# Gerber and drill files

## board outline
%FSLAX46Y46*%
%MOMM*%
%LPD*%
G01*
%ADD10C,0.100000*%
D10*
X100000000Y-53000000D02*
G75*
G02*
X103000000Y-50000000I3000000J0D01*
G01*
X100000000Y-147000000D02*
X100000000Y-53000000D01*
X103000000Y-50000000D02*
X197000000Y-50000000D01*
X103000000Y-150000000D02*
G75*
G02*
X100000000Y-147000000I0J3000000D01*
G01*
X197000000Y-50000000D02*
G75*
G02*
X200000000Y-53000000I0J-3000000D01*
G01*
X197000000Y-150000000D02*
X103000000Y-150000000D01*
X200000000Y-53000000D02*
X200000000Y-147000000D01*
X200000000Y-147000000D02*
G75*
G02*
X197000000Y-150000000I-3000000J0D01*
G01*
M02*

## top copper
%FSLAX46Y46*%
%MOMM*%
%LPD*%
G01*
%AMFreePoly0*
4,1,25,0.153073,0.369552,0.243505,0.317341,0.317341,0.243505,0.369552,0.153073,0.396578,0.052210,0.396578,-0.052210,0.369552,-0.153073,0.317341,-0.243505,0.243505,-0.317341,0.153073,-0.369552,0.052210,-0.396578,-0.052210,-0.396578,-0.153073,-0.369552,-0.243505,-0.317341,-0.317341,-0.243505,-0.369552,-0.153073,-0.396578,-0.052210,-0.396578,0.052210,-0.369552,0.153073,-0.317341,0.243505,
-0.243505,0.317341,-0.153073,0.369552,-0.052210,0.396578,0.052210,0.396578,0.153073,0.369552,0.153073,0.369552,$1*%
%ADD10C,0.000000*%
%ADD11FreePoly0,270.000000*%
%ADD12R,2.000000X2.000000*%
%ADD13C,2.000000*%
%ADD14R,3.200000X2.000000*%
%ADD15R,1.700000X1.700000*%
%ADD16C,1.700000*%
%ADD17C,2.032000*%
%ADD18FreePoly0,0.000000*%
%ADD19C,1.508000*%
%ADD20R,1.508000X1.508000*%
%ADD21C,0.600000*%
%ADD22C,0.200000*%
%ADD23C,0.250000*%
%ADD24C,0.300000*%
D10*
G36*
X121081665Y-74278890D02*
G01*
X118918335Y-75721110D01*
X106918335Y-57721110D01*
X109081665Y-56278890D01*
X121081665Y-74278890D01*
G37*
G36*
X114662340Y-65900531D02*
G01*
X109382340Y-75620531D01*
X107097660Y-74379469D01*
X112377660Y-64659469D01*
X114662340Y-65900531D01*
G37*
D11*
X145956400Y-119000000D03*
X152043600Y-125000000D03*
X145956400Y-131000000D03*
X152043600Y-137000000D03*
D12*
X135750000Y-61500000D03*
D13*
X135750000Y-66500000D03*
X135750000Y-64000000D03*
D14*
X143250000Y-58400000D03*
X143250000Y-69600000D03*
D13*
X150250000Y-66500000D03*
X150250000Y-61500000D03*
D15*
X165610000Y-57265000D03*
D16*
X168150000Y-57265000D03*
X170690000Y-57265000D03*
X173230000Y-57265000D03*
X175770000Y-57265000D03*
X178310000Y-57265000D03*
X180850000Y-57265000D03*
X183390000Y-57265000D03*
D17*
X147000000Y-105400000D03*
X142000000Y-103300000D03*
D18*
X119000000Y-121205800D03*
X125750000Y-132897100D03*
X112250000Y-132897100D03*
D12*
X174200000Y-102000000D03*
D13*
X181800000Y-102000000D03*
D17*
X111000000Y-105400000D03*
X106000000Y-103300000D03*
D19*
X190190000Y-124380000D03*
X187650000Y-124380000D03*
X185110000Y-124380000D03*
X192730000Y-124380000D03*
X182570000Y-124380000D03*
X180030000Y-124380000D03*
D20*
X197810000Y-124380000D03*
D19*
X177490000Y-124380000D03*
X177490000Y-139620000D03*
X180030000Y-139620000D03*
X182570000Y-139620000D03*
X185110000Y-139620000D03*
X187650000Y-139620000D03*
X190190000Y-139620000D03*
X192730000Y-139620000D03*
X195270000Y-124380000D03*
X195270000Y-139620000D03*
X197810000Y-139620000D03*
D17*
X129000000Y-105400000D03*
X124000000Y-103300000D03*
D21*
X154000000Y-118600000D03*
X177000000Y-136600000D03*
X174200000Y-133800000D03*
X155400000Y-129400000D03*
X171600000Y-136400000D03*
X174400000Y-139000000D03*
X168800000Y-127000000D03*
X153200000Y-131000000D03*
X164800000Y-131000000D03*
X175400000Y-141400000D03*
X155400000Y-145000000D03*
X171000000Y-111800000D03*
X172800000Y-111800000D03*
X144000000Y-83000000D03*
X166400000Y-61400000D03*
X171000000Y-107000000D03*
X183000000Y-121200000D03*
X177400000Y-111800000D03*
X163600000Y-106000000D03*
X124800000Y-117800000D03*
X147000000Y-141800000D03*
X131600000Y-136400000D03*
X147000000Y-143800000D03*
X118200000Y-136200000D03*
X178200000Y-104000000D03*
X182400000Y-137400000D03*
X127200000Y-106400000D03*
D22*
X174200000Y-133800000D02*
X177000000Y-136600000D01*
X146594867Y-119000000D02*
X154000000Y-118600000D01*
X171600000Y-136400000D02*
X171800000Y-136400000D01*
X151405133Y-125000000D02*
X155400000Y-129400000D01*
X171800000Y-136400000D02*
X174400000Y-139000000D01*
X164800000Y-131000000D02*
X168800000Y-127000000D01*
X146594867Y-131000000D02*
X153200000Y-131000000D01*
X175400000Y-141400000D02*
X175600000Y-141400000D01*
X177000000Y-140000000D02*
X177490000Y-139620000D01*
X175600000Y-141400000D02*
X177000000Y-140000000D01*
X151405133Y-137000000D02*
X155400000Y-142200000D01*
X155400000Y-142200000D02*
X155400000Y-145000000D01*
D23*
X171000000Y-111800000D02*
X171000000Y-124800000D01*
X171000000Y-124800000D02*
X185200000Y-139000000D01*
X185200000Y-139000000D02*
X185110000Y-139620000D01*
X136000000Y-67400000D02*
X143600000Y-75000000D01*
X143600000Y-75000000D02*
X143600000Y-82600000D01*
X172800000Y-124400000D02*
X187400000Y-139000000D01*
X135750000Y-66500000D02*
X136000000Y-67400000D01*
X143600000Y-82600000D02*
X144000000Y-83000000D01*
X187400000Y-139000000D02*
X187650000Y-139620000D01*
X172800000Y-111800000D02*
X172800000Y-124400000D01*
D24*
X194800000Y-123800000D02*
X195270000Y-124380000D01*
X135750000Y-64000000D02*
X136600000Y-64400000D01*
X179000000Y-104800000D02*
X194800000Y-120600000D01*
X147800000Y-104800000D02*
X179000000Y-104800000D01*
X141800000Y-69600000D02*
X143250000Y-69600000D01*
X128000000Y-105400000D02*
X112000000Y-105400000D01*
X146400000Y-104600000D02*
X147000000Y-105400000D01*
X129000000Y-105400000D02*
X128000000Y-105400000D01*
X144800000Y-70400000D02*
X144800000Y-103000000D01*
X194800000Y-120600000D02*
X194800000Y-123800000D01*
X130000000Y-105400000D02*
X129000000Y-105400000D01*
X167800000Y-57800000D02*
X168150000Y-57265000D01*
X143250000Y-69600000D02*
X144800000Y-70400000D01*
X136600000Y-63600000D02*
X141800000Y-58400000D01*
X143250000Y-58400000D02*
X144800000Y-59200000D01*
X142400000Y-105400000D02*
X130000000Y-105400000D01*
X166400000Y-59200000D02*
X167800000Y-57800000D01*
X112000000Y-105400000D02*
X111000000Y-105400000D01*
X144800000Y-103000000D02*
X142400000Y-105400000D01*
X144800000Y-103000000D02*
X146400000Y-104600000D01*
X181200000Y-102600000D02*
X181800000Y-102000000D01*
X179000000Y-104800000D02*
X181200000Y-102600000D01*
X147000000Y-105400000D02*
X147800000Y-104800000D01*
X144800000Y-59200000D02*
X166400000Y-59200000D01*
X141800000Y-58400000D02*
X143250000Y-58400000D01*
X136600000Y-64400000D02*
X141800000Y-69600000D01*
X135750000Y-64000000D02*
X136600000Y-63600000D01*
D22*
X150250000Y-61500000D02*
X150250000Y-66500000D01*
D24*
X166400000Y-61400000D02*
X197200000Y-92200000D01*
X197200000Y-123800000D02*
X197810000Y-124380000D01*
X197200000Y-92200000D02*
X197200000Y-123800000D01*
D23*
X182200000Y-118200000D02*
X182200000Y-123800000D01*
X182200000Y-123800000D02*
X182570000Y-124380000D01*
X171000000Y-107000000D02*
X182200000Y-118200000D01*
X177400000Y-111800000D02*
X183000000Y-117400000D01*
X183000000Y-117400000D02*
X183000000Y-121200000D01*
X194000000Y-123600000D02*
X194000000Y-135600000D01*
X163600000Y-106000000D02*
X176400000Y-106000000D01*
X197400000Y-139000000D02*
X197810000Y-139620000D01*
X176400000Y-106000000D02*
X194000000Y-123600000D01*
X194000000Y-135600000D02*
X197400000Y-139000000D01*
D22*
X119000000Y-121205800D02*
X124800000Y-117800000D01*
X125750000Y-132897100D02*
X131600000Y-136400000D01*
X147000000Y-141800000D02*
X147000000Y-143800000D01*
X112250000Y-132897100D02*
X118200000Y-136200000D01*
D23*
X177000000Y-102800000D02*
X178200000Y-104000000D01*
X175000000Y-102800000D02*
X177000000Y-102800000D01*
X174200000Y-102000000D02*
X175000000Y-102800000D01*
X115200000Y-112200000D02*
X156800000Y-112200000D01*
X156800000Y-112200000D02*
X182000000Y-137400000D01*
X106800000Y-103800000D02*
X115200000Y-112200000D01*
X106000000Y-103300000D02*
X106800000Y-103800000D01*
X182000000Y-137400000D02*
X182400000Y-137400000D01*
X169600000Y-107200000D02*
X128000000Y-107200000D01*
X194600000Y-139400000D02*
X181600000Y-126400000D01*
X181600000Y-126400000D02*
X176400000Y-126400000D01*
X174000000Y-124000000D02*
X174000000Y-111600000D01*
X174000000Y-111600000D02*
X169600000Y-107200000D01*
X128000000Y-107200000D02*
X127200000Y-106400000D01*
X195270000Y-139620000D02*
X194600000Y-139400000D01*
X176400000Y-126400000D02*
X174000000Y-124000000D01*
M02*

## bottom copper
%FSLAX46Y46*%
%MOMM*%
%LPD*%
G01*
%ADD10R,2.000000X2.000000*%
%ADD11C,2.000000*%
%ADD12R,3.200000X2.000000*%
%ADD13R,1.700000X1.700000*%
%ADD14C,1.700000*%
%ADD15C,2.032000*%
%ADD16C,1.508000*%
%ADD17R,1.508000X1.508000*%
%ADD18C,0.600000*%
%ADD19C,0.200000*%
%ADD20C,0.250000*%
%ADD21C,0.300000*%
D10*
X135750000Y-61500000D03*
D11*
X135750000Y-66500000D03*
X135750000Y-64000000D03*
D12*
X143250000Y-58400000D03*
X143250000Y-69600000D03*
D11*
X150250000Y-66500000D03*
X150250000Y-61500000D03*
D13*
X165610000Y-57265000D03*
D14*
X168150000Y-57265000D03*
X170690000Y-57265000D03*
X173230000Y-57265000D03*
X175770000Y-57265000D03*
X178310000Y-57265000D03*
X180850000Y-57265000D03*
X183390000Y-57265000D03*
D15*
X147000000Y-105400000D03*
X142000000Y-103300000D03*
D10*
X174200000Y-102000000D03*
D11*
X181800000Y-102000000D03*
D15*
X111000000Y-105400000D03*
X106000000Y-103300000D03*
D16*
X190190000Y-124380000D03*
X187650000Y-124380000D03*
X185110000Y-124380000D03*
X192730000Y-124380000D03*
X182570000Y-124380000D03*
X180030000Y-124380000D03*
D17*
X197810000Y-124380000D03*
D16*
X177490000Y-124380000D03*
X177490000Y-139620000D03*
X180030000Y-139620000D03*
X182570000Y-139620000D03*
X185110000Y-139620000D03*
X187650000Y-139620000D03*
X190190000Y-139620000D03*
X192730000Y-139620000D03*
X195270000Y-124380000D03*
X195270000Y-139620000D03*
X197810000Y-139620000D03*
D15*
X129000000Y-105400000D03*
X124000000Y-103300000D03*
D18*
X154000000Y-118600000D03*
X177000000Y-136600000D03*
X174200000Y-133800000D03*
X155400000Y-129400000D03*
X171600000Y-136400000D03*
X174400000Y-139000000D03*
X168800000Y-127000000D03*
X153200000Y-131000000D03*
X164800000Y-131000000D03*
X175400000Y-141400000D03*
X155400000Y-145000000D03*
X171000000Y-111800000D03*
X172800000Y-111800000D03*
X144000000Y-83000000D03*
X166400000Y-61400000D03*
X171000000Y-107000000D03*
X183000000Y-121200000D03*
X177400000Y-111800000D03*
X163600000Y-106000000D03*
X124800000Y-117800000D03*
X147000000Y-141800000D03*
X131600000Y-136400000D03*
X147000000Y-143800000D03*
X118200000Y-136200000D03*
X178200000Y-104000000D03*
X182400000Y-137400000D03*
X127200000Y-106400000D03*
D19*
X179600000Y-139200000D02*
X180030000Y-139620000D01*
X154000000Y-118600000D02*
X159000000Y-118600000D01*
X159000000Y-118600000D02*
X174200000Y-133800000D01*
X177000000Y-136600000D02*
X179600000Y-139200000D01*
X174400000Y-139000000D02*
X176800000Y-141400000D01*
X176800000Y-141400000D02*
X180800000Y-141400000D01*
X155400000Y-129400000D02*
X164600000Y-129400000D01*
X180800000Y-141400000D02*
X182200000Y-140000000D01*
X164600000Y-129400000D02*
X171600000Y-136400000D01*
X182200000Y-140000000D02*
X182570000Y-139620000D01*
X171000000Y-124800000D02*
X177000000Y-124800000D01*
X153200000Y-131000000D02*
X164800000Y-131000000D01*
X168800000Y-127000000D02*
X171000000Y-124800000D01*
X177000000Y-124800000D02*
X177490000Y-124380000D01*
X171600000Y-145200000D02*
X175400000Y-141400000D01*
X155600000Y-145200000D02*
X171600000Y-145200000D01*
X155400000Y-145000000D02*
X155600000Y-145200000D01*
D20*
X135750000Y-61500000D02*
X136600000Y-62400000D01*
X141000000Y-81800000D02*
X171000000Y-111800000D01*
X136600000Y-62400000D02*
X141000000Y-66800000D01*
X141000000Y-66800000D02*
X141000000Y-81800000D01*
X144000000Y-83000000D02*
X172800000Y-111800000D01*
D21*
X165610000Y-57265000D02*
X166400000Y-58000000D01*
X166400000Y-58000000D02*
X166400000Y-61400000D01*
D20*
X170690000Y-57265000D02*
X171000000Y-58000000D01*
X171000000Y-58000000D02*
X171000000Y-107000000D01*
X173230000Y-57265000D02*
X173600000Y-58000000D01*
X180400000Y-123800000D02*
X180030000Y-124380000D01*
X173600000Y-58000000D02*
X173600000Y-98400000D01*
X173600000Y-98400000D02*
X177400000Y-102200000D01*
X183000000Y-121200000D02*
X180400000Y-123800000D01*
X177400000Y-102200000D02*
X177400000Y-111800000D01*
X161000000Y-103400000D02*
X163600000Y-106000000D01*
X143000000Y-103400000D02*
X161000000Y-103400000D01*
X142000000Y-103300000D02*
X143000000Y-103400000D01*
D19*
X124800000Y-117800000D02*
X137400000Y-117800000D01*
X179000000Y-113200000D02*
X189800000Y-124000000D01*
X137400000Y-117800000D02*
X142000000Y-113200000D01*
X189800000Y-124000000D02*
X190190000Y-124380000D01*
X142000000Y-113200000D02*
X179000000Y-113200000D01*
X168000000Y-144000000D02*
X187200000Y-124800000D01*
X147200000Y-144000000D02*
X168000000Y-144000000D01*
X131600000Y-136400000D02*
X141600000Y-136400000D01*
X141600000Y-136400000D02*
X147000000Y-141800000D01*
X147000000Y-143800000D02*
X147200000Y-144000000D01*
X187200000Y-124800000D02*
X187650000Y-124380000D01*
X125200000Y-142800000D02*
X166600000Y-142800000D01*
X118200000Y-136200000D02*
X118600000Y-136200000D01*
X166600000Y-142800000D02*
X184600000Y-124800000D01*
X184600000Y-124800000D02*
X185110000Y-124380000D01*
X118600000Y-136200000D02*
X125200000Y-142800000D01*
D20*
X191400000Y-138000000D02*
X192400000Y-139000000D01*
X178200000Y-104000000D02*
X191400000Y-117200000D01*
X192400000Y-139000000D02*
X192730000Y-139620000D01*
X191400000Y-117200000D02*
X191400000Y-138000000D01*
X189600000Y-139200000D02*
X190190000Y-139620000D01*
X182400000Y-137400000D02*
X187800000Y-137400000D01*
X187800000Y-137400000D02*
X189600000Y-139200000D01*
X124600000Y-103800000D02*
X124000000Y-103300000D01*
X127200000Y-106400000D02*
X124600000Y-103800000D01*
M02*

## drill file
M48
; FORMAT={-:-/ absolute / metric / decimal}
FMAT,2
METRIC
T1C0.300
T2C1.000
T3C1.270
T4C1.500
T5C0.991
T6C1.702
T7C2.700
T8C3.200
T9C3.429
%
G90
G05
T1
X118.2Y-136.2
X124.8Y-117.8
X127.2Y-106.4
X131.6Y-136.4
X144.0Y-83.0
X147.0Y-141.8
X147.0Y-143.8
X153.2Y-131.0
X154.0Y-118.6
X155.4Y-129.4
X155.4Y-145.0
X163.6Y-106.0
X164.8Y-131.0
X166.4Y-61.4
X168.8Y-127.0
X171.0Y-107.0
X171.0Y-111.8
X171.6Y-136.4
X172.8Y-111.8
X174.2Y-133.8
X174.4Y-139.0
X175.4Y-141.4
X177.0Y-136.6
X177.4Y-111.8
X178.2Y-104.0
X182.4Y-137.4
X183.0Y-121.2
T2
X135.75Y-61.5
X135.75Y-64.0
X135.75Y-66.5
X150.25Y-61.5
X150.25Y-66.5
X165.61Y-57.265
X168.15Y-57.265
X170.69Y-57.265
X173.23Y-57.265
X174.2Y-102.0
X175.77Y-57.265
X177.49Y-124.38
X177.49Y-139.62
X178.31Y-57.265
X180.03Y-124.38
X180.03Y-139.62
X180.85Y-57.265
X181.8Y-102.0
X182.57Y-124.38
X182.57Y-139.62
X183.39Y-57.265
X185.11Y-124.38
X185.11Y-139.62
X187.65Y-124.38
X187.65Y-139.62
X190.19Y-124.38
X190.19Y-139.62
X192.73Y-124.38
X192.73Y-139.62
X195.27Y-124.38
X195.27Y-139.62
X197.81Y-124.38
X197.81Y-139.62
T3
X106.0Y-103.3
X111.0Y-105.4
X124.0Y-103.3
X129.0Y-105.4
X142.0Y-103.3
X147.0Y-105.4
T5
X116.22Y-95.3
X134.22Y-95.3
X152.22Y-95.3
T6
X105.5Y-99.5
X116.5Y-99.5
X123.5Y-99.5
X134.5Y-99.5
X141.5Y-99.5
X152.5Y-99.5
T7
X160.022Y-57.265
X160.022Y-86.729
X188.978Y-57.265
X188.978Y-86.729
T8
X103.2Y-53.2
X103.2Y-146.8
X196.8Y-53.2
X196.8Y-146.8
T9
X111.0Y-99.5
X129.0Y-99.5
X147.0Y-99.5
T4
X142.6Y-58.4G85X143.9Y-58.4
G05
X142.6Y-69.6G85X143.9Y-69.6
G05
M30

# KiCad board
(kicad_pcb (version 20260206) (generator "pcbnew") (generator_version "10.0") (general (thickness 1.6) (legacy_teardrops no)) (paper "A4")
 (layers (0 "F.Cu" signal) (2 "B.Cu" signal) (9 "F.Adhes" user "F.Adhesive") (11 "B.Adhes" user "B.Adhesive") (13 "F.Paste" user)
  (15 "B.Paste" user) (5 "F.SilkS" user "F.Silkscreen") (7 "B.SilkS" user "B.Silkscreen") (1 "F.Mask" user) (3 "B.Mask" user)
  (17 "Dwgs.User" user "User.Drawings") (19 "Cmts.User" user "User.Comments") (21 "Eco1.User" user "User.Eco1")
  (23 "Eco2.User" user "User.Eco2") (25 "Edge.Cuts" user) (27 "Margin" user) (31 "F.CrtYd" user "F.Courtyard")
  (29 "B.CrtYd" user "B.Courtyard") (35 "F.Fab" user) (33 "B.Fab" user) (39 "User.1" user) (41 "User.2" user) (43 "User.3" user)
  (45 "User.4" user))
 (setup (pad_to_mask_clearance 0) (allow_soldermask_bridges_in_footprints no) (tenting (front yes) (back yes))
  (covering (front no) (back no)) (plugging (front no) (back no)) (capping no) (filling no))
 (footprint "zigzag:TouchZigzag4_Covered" (layer "F.Cu") (at 149 128 -90)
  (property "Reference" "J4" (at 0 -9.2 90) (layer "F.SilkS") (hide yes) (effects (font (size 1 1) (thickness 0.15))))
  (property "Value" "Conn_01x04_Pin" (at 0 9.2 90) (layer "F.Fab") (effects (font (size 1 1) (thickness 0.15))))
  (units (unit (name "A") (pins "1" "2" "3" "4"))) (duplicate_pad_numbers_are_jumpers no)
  (pad "1" smd custom (at -9 3.0436 270) (size 0.8 0.8) (layers "F.Cu") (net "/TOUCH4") (options (clearance outline) (anchor circle))
   (primitives))
  (pad "2" smd custom (at -3 -3.0436 270) (size 0.8 0.8) (layers "F.Cu") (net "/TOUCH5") (options (clearance outline) (anchor circle))
   (primitives))
  (pad "3" smd custom (at 3 3.0436 270) (size 0.8 0.8) (layers "F.Cu") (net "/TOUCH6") (options (clearance outline) (anchor circle))
   (primitives))
  (pad "4" smd custom (at 9 -3.0436 270) (size 0.8 0.8) (layers "F.Cu") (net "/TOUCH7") (options (clearance outline) (anchor circle))
   (primitives)))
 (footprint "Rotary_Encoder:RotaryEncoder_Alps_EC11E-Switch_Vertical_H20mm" (layer "F.Cu") (at 135.75 61.5)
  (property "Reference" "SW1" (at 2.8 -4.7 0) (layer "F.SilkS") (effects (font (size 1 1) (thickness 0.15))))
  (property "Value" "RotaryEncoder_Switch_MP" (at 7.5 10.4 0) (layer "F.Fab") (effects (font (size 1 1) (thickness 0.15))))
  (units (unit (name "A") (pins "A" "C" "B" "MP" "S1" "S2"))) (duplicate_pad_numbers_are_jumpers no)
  (pad "A" thru_hole rect (at 0 0) (size 2 2) (drill 1) (layers "*.Cu" "*.Mask") (remove_unused_layers no) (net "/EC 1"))
  (pad "B" thru_hole circle (at 0 5) (size 2 2) (drill 1) (layers "*.Cu" "*.Mask") (remove_unused_layers no) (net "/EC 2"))
  (pad "C" thru_hole circle (at 0 2.5) (size 2 2) (drill 1) (layers "*.Cu" "*.Mask") (remove_unused_layers no) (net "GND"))
  (pad "MP" thru_hole rect (at 7.5 -3.1) (size 3.2 2) (drill oval 2.8 1.5) (layers "*.Cu" "*.Mask") (remove_unused_layers no) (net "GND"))
  (pad "MP" thru_hole rect (at 7.5 8.1) (size 3.2 2) (drill oval 2.8 1.5) (layers "*.Cu" "*.Mask") (remove_unused_layers no) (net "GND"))
  (pad "S1" thru_hole circle (at 14.5 5) (size 2 2) (drill 1) (layers "*.Cu" "*.Mask") (remove_unused_layers no)
   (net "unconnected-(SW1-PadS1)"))
  (pad "S2" thru_hole circle (at 14.5 0) (size 2 2) (drill 1) (layers "*.Cu" "*.Mask") (remove_unused_layers no)
   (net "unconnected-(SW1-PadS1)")))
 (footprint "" (layer "F.Cu") (at 196.8 53.2)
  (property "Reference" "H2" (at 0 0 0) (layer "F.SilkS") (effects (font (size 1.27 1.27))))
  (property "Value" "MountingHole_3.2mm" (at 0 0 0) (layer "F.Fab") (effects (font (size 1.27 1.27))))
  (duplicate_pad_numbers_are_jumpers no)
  (pad "" np_thru_hole circle (at 0 0) (size 3.2 3.2) (drill 3.2) (layers "*.Cu" "*.Mask")))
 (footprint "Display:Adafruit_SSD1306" (layer "F.Cu") (at 165.61 57.265)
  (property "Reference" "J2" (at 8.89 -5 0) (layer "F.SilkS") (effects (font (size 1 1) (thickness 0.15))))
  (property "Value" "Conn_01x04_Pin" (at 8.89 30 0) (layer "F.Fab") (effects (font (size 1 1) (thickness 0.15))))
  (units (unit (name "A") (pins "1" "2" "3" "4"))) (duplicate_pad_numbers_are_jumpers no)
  (pad "" np_thru_hole circle (at -5.588 0) (size 2.7 2.7) (drill 2.7) (layers "*.Cu" "*.Mask"))
  (pad "" np_thru_hole circle (at -5.588 29.464) (size 2.7 2.7) (drill 2.7) (layers "*.Cu" "*.Mask"))
  (pad "" np_thru_hole circle (at 23.368 0) (size 2.7 2.7) (drill 2.7) (layers "*.Cu" "*.Mask"))
  (pad "" np_thru_hole circle (at 23.368 29.464) (size 2.7 2.7) (drill 2.7) (layers "*.Cu" "*.Mask"))
  (pad "1" thru_hole rect (at 0 0) (size 1.7 1.7) (drill 1) (layers "*.Cu" "*.Mask") (remove_unused_layers no) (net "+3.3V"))
  (pad "2" thru_hole circle (at 2.54 0) (size 1.7 1.7) (drill 1) (layers "*.Cu" "*.Mask") (remove_unused_layers no) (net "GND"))
  (pad "3" thru_hole circle (at 5.08 0) (size 1.7 1.7) (drill 1) (layers "*.Cu" "*.Mask") (remove_unused_layers no) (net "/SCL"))
  (pad "4" thru_hole circle (at 7.62 0) (size 1.7 1.7) (drill 1) (layers "*.Cu" "*.Mask") (remove_unused_layers no) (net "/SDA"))
  (pad "5" thru_hole circle (at 10.16 0) (size 1.7 1.7) (drill 1) (layers "*.Cu" "*.Mask") (remove_unused_layers no))
  (pad "6" thru_hole circle (at 12.7 0) (size 1.7 1.7) (drill 1) (layers "*.Cu" "*.Mask") (remove_unused_layers no))
  (pad "7" thru_hole circle (at 15.24 0) (size 1.7 1.7) (drill 1) (layers "*.Cu" "*.Mask") (remove_unused_layers no))
  (pad "8" thru_hole circle (at 17.78 0) (size 1.7 1.7) (drill 1) (layers "*.Cu" "*.Mask") (remove_unused_layers no)))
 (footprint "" (layer "F.Cu") (at 103.2 146.8)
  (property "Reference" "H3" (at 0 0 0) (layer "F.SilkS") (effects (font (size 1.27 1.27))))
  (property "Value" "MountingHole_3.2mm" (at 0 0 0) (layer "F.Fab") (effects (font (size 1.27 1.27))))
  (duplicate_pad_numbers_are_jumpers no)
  (pad "" np_thru_hole circle (at 0 0) (size 3.2 3.2) (drill 3.2) (layers "*.Cu" "*.Mask")))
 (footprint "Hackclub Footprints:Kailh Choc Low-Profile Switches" (layer "F.Cu") (at 147 99.5)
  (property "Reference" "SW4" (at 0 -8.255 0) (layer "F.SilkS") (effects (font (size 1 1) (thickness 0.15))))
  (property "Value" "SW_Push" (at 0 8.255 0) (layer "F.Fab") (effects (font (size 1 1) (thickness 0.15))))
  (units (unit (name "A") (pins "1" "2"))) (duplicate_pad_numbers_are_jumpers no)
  (pad "" np_thru_hole circle (at -5.5 0) (size 1.7018 1.7018) (drill 1.7018) (layers "*.Cu" "*.Mask"))
  (pad "" np_thru_hole circle (at 0 0) (size 3.429 3.429) (drill 3.429) (layers "*.Cu" "*.Mask"))
  (pad "" np_thru_hole circle (at 5.22 -4.2) (size 0.9906 0.9906) (drill 0.9906) (layers "*.Cu" "*.Mask"))
  (pad "" np_thru_hole circle (at 5.5 0) (size 1.7018 1.7018) (drill 1.7018) (layers "*.Cu" "*.Mask"))
  (pad "1" thru_hole circle (at 0 5.9) (size 2.032 2.032) (drill 1.27) (layers "*.Cu" "*.Mask") (remove_unused_layers no) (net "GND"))
  (pad "2" thru_hole circle (at -5 3.8) (size 2.032 2.032) (drill 1.27) (layers "*.Cu" "*.Mask") (remove_unused_layers no) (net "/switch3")))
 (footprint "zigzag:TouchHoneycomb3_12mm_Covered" (layer "F.Cu") (at 119 129)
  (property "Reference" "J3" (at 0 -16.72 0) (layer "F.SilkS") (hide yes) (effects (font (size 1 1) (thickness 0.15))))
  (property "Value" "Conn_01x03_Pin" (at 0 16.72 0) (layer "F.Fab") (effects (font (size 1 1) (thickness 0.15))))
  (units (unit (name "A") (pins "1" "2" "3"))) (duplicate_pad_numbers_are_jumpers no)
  (pad "1" smd custom (at 0 -7.7942) (size 0.8 0.8) (layers "F.Cu") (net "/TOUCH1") (options (clearance outline) (anchor circle))
   (primitives))
  (pad "2" smd custom (at 6.75 3.8971) (size 0.8 0.8) (layers "F.Cu") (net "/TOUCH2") (options (clearance outline) (anchor circle))
   (primitives))
  (pad "3" smd custom (at -6.75 3.8971) (size 0.8 0.8) (layers "F.Cu") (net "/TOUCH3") (options (clearance outline) (anchor circle))
   (primitives)))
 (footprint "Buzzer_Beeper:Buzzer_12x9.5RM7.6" (layer "F.Cu") (at 174.2 102)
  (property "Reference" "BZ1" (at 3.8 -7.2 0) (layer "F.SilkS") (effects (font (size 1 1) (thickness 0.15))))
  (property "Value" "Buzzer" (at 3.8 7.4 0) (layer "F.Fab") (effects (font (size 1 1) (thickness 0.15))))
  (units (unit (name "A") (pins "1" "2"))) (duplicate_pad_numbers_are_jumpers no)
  (pad "1" thru_hole rect (at 0 0) (size 2 2) (drill 1) (layers "*.Cu" "*.Mask") (remove_unused_layers no) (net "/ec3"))
  (pad "2" thru_hole circle (at 7.6 0) (size 2 2) (drill 1) (layers "*.Cu" "*.Mask") (remove_unused_layers no) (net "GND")))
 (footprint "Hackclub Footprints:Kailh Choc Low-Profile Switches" (layer "F.Cu") (at 111 99.5)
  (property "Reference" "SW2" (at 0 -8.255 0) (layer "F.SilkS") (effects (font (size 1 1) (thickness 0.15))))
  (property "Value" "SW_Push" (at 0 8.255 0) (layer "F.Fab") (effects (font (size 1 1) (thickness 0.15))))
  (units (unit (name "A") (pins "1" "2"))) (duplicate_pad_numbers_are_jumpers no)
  (pad "" np_thru_hole circle (at -5.5 0) (size 1.7018 1.7018) (drill 1.7018) (layers "*.Cu" "*.Mask"))
  (pad "" np_thru_hole circle (at 0 0) (size 3.429 3.429) (drill 3.429) (layers "*.Cu" "*.Mask"))
  (pad "" np_thru_hole circle (at 5.22 -4.2) (size 0.9906 0.9906) (drill 0.9906) (layers "*.Cu" "*.Mask"))
  (pad "" np_thru_hole circle (at 5.5 0) (size 1.7018 1.7018) (drill 1.7018) (layers "*.Cu" "*.Mask"))
  (pad "1" thru_hole circle (at 0 5.9) (size 2.032 2.032) (drill 1.27) (layers "*.Cu" "*.Mask") (remove_unused_layers no) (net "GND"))
  (pad "2" thru_hole circle (at -5 3.8) (size 2.032 2.032) (drill 1.27) (layers "*.Cu" "*.Mask") (remove_unused_layers no) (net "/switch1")))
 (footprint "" (layer "F.Cu") (at 103.2 53.2)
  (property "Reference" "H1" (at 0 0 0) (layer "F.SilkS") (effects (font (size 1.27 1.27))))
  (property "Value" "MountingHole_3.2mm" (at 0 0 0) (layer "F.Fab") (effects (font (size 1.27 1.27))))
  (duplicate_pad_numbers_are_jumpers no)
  (pad "" np_thru_hole circle (at 0 0) (size 3.2 3.2) (drill 3.2) (layers "*.Cu" "*.Mask")))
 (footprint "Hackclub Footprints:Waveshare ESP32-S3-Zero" (layer "F.Cu") (at 187.65 132 -90)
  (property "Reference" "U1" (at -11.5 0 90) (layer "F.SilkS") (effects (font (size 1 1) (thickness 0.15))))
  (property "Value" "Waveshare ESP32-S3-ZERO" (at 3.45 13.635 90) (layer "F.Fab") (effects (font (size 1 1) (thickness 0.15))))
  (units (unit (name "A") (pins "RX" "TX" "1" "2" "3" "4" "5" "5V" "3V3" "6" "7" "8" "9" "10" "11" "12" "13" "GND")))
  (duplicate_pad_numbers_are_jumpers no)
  (pad "1" thru_hole circle (at -7.62 -2.54 270) (size 1.508 1.508) (drill 1) (layers "*.Cu" "*.Mask") (remove_unused_layers no)
   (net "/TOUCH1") (solder_mask_margin 0.102))
  (pad "2" thru_hole circle (at -7.62 0 270) (size 1.508 1.508) (drill 1) (layers "*.Cu" "*.Mask") (remove_unused_layers no) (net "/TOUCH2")
   (solder_mask_margin 0.102))
  (pad "3" thru_hole circle (at -7.62 2.54 270) (size 1.508 1.508) (drill 1) (layers "*.Cu" "*.Mask") (remove_unused_layers no)
   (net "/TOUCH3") (solder_mask_margin 0.102))
  (pad "3V3" thru_hole circle (at -7.62 -5.08 270) (size 1.508 1.508) (drill 1) (layers "*.Cu" "*.Mask") (remove_unused_layers no)
   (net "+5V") (solder_mask_margin 0.102))
  (pad "4" thru_hole circle (at -7.62 5.08 270) (size 1.508 1.508) (drill 1) (layers "*.Cu" "*.Mask") (remove_unused_layers no) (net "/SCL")
   (solder_mask_margin 0.102))
  (pad "5" thru_hole circle (at -7.62 7.62 270) (size 1.508 1.508) (drill 1) (layers "*.Cu" "*.Mask") (remove_unused_layers no) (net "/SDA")
   (solder_mask_margin 0.102))
  (pad "5V" thru_hole rect (at -7.62 -10.16 270) (size 1.508 1.508) (drill 1) (layers "*.Cu" "*.Mask") (remove_unused_layers no)
   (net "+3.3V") (solder_mask_margin 0.102))
  (pad "6" thru_hole circle (at -7.62 10.16 270) (size 1.508 1.508) (drill 1) (layers "*.Cu" "*.Mask") (remove_unused_layers no)
   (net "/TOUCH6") (solder_mask_margin 0.102))
  (pad "7" thru_hole circle (at 7.62 10.16 270) (size 1.508 1.508) (drill 1) (layers "*.Cu" "*.Mask") (remove_unused_layers no)
   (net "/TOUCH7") (solder_mask_margin 0.102))
  (pad "8" thru_hole circle (at 7.62 7.62 270) (size 1.508 1.508) (drill 1) (layers "*.Cu" "*.Mask") (remove_unused_layers no)
   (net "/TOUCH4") (solder_mask_margin 0.102))
  (pad "9" thru_hole circle (at 7.62 5.08 270) (size 1.508 1.508) (drill 1) (layers "*.Cu" "*.Mask") (remove_unused_layers no)
   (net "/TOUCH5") (solder_mask_margin 0.102))
  (pad "10" thru_hole circle (at 7.62 2.54 270) (size 1.508 1.508) (drill 1) (layers "*.Cu" "*.Mask") (remove_unused_layers no)
   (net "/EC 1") (solder_mask_margin 0.102))
  (pad "11" thru_hole circle (at 7.62 0 270) (size 1.508 1.508) (drill 1) (layers "*.Cu" "*.Mask") (remove_unused_layers no) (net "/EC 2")
   (solder_mask_margin 0.102))
  (pad "12" thru_hole circle (at 7.62 -2.54 270) (size 1.508 1.508) (drill 1) (layers "*.Cu" "*.Mask") (remove_unused_layers no)
   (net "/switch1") (solder_mask_margin 0.102))
  (pad "13" thru_hole circle (at 7.62 -5.08 270) (size 1.508 1.508) (drill 1) (layers "*.Cu" "*.Mask") (remove_unused_layers no)
   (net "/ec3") (solder_mask_margin 0.102))
  (pad "GND" thru_hole circle (at -7.62 -7.62 270) (size 1.508 1.508) (drill 1) (layers "*.Cu" "*.Mask") (remove_unused_layers no)
   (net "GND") (solder_mask_margin 0.102))
  (pad "RX" thru_hole circle (at 7.62 -7.62 270) (size 1.508 1.508) (drill 1) (layers "*.Cu" "*.Mask") (remove_unused_layers no)
   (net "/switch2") (solder_mask_margin 0.102))
  (pad "TX" thru_hole circle (at 7.62 -10.16 270) (size 1.508 1.508) (drill 1) (layers "*.Cu" "*.Mask") (remove_unused_layers no)
   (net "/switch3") (solder_mask_margin 0.102)))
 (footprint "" (layer "F.Cu") (at 196.8 146.8)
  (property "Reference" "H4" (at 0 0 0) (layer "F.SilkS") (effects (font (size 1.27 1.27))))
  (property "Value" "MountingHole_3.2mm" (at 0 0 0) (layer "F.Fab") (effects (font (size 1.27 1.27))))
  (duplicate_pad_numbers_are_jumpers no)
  (pad "" np_thru_hole circle (at 0 0) (size 3.2 3.2) (drill 3.2) (layers "*.Cu" "*.Mask")))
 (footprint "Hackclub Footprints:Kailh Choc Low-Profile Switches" (layer "F.Cu") (at 129 99.5)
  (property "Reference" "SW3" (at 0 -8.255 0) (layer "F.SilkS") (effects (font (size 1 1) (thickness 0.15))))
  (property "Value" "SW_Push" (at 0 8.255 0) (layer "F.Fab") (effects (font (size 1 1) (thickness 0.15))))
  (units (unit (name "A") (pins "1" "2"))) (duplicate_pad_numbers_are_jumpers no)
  (pad "" np_thru_hole circle (at -5.5 0) (size 1.7018 1.7018) (drill 1.7018) (layers "*.Cu" "*.Mask"))
  (pad "" np_thru_hole circle (at 0 0) (size 3.429 3.429) (drill 3.429) (layers "*.Cu" "*.Mask"))
  (pad "" np_thru_hole circle (at 5.22 -4.2) (size 0.9906 0.9906) (drill 0.9906) (layers "*.Cu" "*.Mask"))
  (pad "" np_thru_hole circle (at 5.5 0) (size 1.7018 1.7018) (drill 1.7018) (layers "*.Cu" "*.Mask"))
  (pad "1" thru_hole circle (at 0 5.9) (size 2.032 2.032) (drill 1.27) (layers "*.Cu" "*.Mask") (remove_unused_layers no) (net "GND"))
  (pad "2" thru_hole circle (at -5 3.8) (size 2.032 2.032) (drill 1.27) (layers "*.Cu" "*.Mask") (remove_unused_layers no) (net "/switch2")))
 (gr_poly
  (pts (xy 106.918335 57.72111) (xy 118.918335 75.72111) (xy 121.081665 74.27889) (xy 109.081665 56.27889))
  (stroke (width 0) (type default)) (fill yes) (layer "F.Cu"))
 (gr_poly
  (pts (xy 112.37766 64.659469) (xy 107.09766 74.379469) (xy 109.38234 75.620531) (xy 114.66234 65.900531))
  (stroke (width 0) (type default)) (fill yes) (layer "F.Cu"))
 (gr_arc (start 100 53) (mid 100.87868 50.87868) (end 103 50) (stroke (width 0.1) (type default)) (layer "Edge.Cuts"))
 (gr_line (start 100 147) (end 100 53) (stroke (width 0.1) (type default)) (layer "Edge.Cuts"))
 (gr_line (start 103 50) (end 197 50) (stroke (width 0.1) (type default)) (layer "Edge.Cuts"))
 (gr_arc (start 103 150) (mid 100.87868 149.12132) (end 100 147) (stroke (width 0.1) (type default)) (layer "Edge.Cuts"))
 (gr_arc (start 197 50) (mid 199.12132 50.87868) (end 200 53) (stroke (width 0.1) (type default)) (layer "Edge.Cuts"))
 (gr_line (start 197 150) (end 103 150) (stroke (width 0.1) (type default)) (layer "Edge.Cuts"))
 (gr_line (start 200 53) (end 200 147) (stroke (width 0.1) (type default)) (layer "Edge.Cuts"))
 (gr_arc (start 200 147) (mid 199.12132 149.12132) (end 197 150) (stroke (width 0.1) (type default)) (layer "Edge.Cuts"))
 (segment (start 174.2 133.8) (end 177 136.6) (width 0.2) (layer "F.Cu") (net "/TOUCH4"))
 (segment (start 146.594867 119) (end 154 118.6) (width 0.2) (layer "F.Cu") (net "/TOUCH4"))
 (via (at 154 118.6) (size 0.6) (drill 0.3) (layers "F.Cu" "B.Cu") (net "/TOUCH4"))
 (via (at 177 136.6) (size 0.6) (drill 0.3) (layers "F.Cu" "B.Cu") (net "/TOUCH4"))
 (via (at 174.2 133.8) (size 0.6) (drill 0.3) (layers "F.Cu" "B.Cu") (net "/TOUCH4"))
 (segment (start 179.6 139.2) (end 180.03 139.62) (width 0.2) (layer "B.Cu") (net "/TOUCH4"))
 (segment (start 154 118.6) (end 159 118.6) (width 0.2) (layer "B.Cu") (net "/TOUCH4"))
 (segment (start 159 118.6) (end 174.2 133.8) (width 0.2) (layer "B.Cu") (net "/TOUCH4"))
 (segment (start 177 136.6) (end 179.6 139.2) (width 0.2) (layer "B.Cu") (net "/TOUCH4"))
 (segment (start 171.6 136.4) (end 171.8 136.4) (width 0.2) (layer "F.Cu") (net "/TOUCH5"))
 (segment (start 151.405133 125) (end 155.4 129.4) (width 0.2) (layer "F.Cu") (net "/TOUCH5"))
 (segment (start 171.8 136.4) (end 174.4 139) (width 0.2) (layer "F.Cu") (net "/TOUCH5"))
 (via (at 155.4 129.4) (size 0.6) (drill 0.3) (layers "F.Cu" "B.Cu") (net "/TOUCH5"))
 (via (at 171.6 136.4) (size 0.6) (drill 0.3) (layers "F.Cu" "B.Cu") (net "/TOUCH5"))
 (via (at 174.4 139) (size 0.6) (drill 0.3) (layers "F.Cu" "B.Cu") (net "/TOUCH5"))
 (segment (start 174.4 139) (end 176.8 141.4) (width 0.2) (layer "B.Cu") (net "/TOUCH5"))
 (segment (start 176.8 141.4) (end 180.8 141.4) (width 0.2) (layer "B.Cu") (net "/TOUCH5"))
 (segment (start 155.4 129.4) (end 164.6 129.4) (width 0.2) (layer "B.Cu") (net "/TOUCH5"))
 (segment (start 180.8 141.4) (end 182.2 140) (width 0.2) (layer "B.Cu") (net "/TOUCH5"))
 (segment (start 164.6 129.4) (end 171.6 136.4) (width 0.2) (layer "B.Cu") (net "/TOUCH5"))
 (segment (start 182.2 140) (end 182.57 139.62) (width 0.2) (layer "B.Cu") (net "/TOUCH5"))
 (segment (start 164.8 131) (end 168.8 127) (width 0.2) (layer "F.Cu") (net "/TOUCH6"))
 (segment (start 146.594867 131) (end 153.2 131) (width 0.2) (layer "F.Cu") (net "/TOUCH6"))
 (via (at 168.8 127) (size 0.6) (drill 0.3) (layers "F.Cu" "B.Cu") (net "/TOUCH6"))
 (via (at 153.2 131) (size 0.6) (drill 0.3) (layers "F.Cu" "B.Cu") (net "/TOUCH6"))
 (via (at 164.8 131) (size 0.6) (drill 0.3) (layers "F.Cu" "B.Cu") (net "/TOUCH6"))
 (segment (start 171 124.8) (end 177 124.8) (width 0.2) (layer "B.Cu") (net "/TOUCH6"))
 (segment (start 153.2 131) (end 164.8 131) (width 0.2) (layer "B.Cu") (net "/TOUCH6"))
 (segment (start 168.8 127) (end 171 124.8) (width 0.2) (layer "B.Cu") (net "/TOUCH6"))
 (segment (start 177 124.8) (end 177.49 124.38) (width 0.2) (layer "B.Cu") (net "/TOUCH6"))
 (segment (start 175.4 141.4) (end 175.6 141.4) (width 0.2) (layer "F.Cu") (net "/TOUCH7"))
 (segment (start 177 140) (end 177.49 139.62) (width 0.2) (layer "F.Cu") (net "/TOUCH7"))
 (segment (start 175.6 141.4) (end 177 140) (width 0.2) (layer "F.Cu") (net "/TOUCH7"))
 (segment (start 151.405133 137) (end 155.4 142.2) (width 0.2) (layer "F.Cu") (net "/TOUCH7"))
 (segment (start 155.4 142.2) (end 155.4 145) (width 0.2) (layer "F.Cu") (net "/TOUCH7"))
 (via (at 175.4 141.4) (size 0.6) (drill 0.3) (layers "F.Cu" "B.Cu") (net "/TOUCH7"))
 (via (at 155.4 145) (size 0.6) (drill 0.3) (layers "F.Cu" "B.Cu") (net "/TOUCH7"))
 (segment (start 171.6 145.2) (end 175.4 141.4) (width 0.2) (layer "B.Cu") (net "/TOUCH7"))
 (segment (start 155.6 145.2) (end 171.6 145.2) (width 0.2) (layer "B.Cu") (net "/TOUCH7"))
 (segment (start 155.4 145) (end 155.6 145.2) (width 0.2) (layer "B.Cu") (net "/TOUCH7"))
 (segment (start 171 111.8) (end 171 124.8) (width 0.25) (layer "F.Cu") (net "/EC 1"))
 (segment (start 171 124.8) (end 185.2 139) (width 0.25) (layer "F.Cu") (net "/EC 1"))
 (segment (start 185.2 139) (end 185.11 139.62) (width 0.25) (layer "F.Cu") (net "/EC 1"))
 (via (at 171 111.8) (size 0.6) (drill 0.3) (layers "F.Cu" "B.Cu") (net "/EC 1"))
 (segment (start 135.75 61.5) (end 136.6 62.4) (width 0.25) (layer "B.Cu") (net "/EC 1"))
 (segment (start 141 81.8) (end 171 111.8) (width 0.25) (layer "B.Cu") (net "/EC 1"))
 (segment (start 136.6 62.4) (end 141 66.8) (width 0.25) (layer "B.Cu") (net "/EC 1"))
 (segment (start 141 66.8) (end 141 81.8) (width 0.25) (layer "B.Cu") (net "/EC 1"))
 (segment (start 136 67.4) (end 143.6 75) (width 0.25) (layer "F.Cu") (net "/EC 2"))
 (segment (start 143.6 75) (end 143.6 82.6) (width 0.25) (layer "F.Cu") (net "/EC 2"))
 (segment (start 172.8 124.4) (end 187.4 139) (width 0.25) (layer "F.Cu") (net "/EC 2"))
 (segment (start 135.75 66.5) (end 136 67.4) (width 0.25) (layer "F.Cu") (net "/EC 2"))
 (segment (start 143.6 82.6) (end 144 83) (width 0.25) (layer "F.Cu") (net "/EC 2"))
 (segment (start 187.4 139) (end 187.65 139.62) (width 0.25) (layer "F.Cu") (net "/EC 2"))
 (segment (start 172.8 111.8) (end 172.8 124.4) (width 0.25) (layer "F.Cu") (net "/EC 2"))
 (via (at 172.8 111.8) (size 0.6) (drill 0.3) (layers "F.Cu" "B.Cu") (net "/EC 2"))
 (via (at 144 83) (size 0.6) (drill 0.3) (layers "F.Cu" "B.Cu") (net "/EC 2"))
 (segment (start 144 83) (end 172.8 111.8) (width 0.25) (layer "B.Cu") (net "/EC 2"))
 (segment (start 194.8 123.8) (end 195.27 124.38) (width 0.3) (layer "F.Cu") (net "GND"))
 (segment (start 135.75 64) (end 136.6 64.4) (width 0.3) (layer "F.Cu") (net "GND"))
 (segment (start 179 104.8) (end 194.8 120.6) (width 0.3) (layer "F.Cu") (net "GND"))
 (segment (start 147.8 104.8) (end 179 104.8) (width 0.3) (layer "F.Cu") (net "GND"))
 (segment (start 141.8 69.6) (end 143.25 69.6) (width 0.3) (layer "F.Cu") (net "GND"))
 (segment (start 128 105.4) (end 112 105.4) (width 0.3) (layer "F.Cu") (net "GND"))
 (segment (start 146.4 104.6) (end 147 105.4) (width 0.3) (layer "F.Cu") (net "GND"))
 (segment (start 129 105.4) (end 128 105.4) (width 0.3) (layer "F.Cu") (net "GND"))
 (segment (start 144.8 70.4) (end 144.8 103) (width 0.3) (layer "F.Cu") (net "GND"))
 (segment (start 194.8 120.6) (end 194.8 123.8) (width 0.3) (layer "F.Cu") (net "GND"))
 (segment (start 130 105.4) (end 129 105.4) (width 0.3) (layer "F.Cu") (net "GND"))
 (segment (start 167.8 57.8) (end 168.15 57.265) (width 0.3) (layer "F.Cu") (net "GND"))
 (segment (start 143.25 69.6) (end 144.8 70.4) (width 0.3) (layer "F.Cu") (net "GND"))
 (segment (start 136.6 63.6) (end 141.8 58.4) (width 0.3) (layer "F.Cu") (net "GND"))
 (segment (start 143.25 58.4) (end 144.8 59.2) (width 0.3) (layer "F.Cu") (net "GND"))
 (segment (start 142.4 105.4) (end 130 105.4) (width 0.3) (layer "F.Cu") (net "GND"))
 (segment (start 166.4 59.2) (end 167.8 57.8) (width 0.3) (layer "F.Cu") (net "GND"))
 (segment (start 112 105.4) (end 111 105.4) (width 0.3) (layer "F.Cu") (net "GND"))
 (segment (start 144.8 103) (end 142.4 105.4) (width 0.3) (layer "F.Cu") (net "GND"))
 (segment (start 144.8 103) (end 146.4 104.6) (width 0.3) (layer "F.Cu") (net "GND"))
 (segment (start 181.2 102.6) (end 181.8 102) (width 0.3) (layer "F.Cu") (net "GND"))
 (segment (start 179 104.8) (end 181.2 102.6) (width 0.3) (layer "F.Cu") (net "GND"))
 (segment (start 147 105.4) (end 147.8 104.8) (width 0.3) (layer "F.Cu") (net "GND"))
 (segment (start 144.8 59.2) (end 166.4 59.2) (width 0.3) (layer "F.Cu") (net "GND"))
 (segment (start 141.8 58.4) (end 143.25 58.4) (width 0.3) (layer "F.Cu") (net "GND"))
 (segment (start 136.6 64.4) (end 141.8 69.6) (width 0.3) (layer "F.Cu") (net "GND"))
 (segment (start 135.75 64) (end 136.6 63.6) (width 0.3) (layer "F.Cu") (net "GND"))
 (segment (start 150.25 61.5) (end 150.25 66.5) (width 0.2) (layer "F.Cu") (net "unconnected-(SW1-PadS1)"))
 (segment (start 166.4 61.4) (end 197.2 92.2) (width 0.3) (layer "F.Cu") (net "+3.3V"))
 (segment (start 197.2 123.8) (end 197.81 124.38) (width 0.3) (layer "F.Cu") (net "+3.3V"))
 (segment (start 197.2 92.2) (end 197.2 123.8) (width 0.3) (layer "F.Cu") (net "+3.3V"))
 (via (at 166.4 61.4) (size 0.6) (drill 0.3) (layers "F.Cu" "B.Cu") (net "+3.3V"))
 (segment (start 165.61 57.265) (end 166.4 58) (width 0.3) (layer "B.Cu") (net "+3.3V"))
 (segment (start 166.4 58) (end 166.4 61.4) (width 0.3) (layer "B.Cu") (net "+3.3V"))
 (segment (start 182.2 118.2) (end 182.2 123.8) (width 0.25) (layer "F.Cu") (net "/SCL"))
 (segment (start 182.2 123.8) (end 182.57 124.38) (width 0.25) (layer "F.Cu") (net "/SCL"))
 (segment (start 171 107) (end 182.2 118.2) (width 0.25) (layer "F.Cu") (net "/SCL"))
 (via (at 171 107) (size 0.6) (drill 0.3) (layers "F.Cu" "B.Cu") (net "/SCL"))
 (segment (start 170.69 57.265) (end 171 58) (width 0.25) (layer "B.Cu") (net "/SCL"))
 (segment (start 171 58) (end 171 107) (width 0.25) (layer "B.Cu") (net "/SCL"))
 (segment (start 177.4 111.8) (end 183 117.4) (width 0.25) (layer "F.Cu") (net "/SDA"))
 (segment (start 183 117.4) (end 183 121.2) (width 0.25) (layer "F.Cu") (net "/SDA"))
 (via (at 183 121.2) (size 0.6) (drill 0.3) (layers "F.Cu" "B.Cu") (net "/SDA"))
 (via (at 177.4 111.8) (size 0.6) (drill 0.3) (layers "F.Cu" "B.Cu") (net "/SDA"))
 (segment (start 173.23 57.265) (end 173.6 58) (width 0.25) (layer "B.Cu") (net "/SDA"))
 (segment (start 180.4 123.8) (end 180.03 124.38) (width 0.25) (layer "B.Cu") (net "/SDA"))
 (segment (start 173.6 58) (end 173.6 98.4) (width 0.25) (layer "B.Cu") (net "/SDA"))
 (segment (start 173.6 98.4) (end 177.4 102.2) (width 0.25) (layer "B.Cu") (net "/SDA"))
 (segment (start 183 121.2) (end 180.4 123.8) (width 0.25) (layer "B.Cu") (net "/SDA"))
 (segment (start 177.4 102.2) (end 177.4 111.8) (width 0.25) (layer "B.Cu") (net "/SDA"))
 (segment (start 194 123.6) (end 194 135.6) (width 0.25) (layer "F.Cu") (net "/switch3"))
 (segment (start 163.6 106) (end 176.4 106) (width 0.25) (layer "F.Cu") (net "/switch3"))
 (segment (start 197.4 139) (end 197.81 139.62) (width 0.25) (layer "F.Cu") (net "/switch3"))
 (segment (start 176.4 106) (end 194 123.6) (width 0.25) (layer "F.Cu") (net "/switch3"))
 (segment (start 194 135.6) (end 197.4 139) (width 0.25) (layer "F.Cu") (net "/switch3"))
 (via (at 163.6 106) (size 0.6) (drill 0.3) (layers "F.Cu" "B.Cu") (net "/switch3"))
 (segment (start 161 103.4) (end 163.6 106) (width 0.25) (layer "B.Cu") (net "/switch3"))
 (segment (start 143 103.4) (end 161 103.4) (width 0.25) (layer "B.Cu") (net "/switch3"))
 (segment (start 142 103.3) (end 143 103.4) (width 0.25) (layer "B.Cu") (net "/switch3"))
 (segment (start 119 121.2058) (end 124.8 117.8) (width 0.2) (layer "F.Cu") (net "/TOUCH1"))
 (via (at 124.8 117.8) (size 0.6) (drill 0.3) (layers "F.Cu" "B.Cu") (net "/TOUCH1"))
 (segment (start 124.8 117.8) (end 137.4 117.8) (width 0.2) (layer "B.Cu") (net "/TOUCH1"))
 (segment (start 179 113.2) (end 189.8 124) (width 0.2) (layer "B.Cu") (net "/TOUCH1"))
 (segment (start 137.4 117.8) (end 142 113.2) (width 0.2) (layer "B.Cu") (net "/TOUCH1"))
 (segment (start 189.8 124) (end 190.19 124.38) (width 0.2) (layer "B.Cu") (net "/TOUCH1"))
 (segment (start 142 113.2) (end 179 113.2) (width 0.2) (layer "B.Cu") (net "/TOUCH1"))
 (segment (start 125.75 132.8971) (end 131.6 136.4) (width 0.2) (layer "F.Cu") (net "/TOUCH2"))
 (segment (start 147 141.8) (end 147 143.8) (width 0.2) (layer "F.Cu") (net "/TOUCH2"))
 (via (at 147 141.8) (size 0.6) (drill 0.3) (layers "F.Cu" "B.Cu") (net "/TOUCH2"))
 (via (at 131.6 136.4) (size 0.6) (drill 0.3) (layers "F.Cu" "B.Cu") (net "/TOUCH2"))
 (via (at 147 143.8) (size 0.6) (drill 0.3) (layers "F.Cu" "B.Cu") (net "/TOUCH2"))
 (segment (start 168 144) (end 187.2 124.8) (width 0.2) (layer "B.Cu") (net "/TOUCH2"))
 (segment (start 147.2 144) (end 168 144) (width 0.2) (layer "B.Cu") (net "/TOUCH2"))
 (segment (start 131.6 136.4) (end 141.6 136.4) (width 0.2) (layer "B.Cu") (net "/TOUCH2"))
 (segment (start 141.6 136.4) (end 147 141.8) (width 0.2) (layer "B.Cu") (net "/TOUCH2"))
 (segment (start 147 143.8) (end 147.2 144) (width 0.2) (layer "B.Cu") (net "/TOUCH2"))
 (segment (start 187.2 124.8) (end 187.65 124.38) (width 0.2) (layer "B.Cu") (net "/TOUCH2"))
 (segment (start 112.25 132.8971) (end 118.2 136.2) (width 0.2) (layer "F.Cu") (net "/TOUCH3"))
 (via (at 118.2 136.2) (size 0.6) (drill 0.3) (layers "F.Cu" "B.Cu") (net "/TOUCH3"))
 (segment (start 125.2 142.8) (end 166.6 142.8) (width 0.2) (layer "B.Cu") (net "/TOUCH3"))
 (segment (start 118.2 136.2) (end 118.6 136.2) (width 0.2) (layer "B.Cu") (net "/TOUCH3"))
 (segment (start 166.6 142.8) (end 184.6 124.8) (width 0.2) (layer "B.Cu") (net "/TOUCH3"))
 (segment (start 184.6 124.8) (end 185.11 124.38) (width 0.2) (layer "B.Cu") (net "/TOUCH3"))
 (segment (start 118.6 136.2) (end 125.2 142.8) (width 0.2) (layer "B.Cu") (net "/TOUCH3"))
 (segment (start 177 102.8) (end 178.2 104) (width 0.25) (layer "F.Cu") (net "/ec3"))
 (segment (start 175 102.8) (end 177 102.8) (width 0.25) (layer "F.Cu") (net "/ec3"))
 (segment (start 174.2 102) (end 175 102.8) (width 0.25) (layer "F.Cu") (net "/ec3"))
 (via (at 178.2 104) (size 0.6) (drill 0.3) (layers "F.Cu" "B.Cu") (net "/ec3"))
 (segment (start 191.4 138) (end 192.4 139) (width 0.25) (layer "B.Cu") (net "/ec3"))
 (segment (start 178.2 104) (end 191.4 117.2) (width 0.25) (layer "B.Cu") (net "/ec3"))
 (segment (start 192.4 139) (end 192.73 139.62) (width 0.25) (layer "B.Cu") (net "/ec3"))
 (segment (start 191.4 117.2) (end 191.4 138) (width 0.25) (layer "B.Cu") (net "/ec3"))
 (segment (start 115.2 112.2) (end 156.8 112.2) (width 0.25) (layer "F.Cu") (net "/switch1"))
 (segment (start 156.8 112.2) (end 182 137.4) (width 0.25) (layer "F.Cu") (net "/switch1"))
 (segment (start 106.8 103.8) (end 115.2 112.2) (width 0.25) (layer "F.Cu") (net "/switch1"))
 (segment (start 106 103.3) (end 106.8 103.8) (width 0.25) (layer "F.Cu") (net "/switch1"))
 (segment (start 182 137.4) (end 182.4 137.4) (width 0.25) (layer "F.Cu") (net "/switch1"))
 (via (at 182.4 137.4) (size 0.6) (drill 0.3) (layers "F.Cu" "B.Cu") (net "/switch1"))
 (segment (start 189.6 139.2) (end 190.19 139.62) (width 0.25) (layer "B.Cu") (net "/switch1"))
 (segment (start 182.4 137.4) (end 187.8 137.4) (width 0.25) (layer "B.Cu") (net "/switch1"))
 (segment (start 187.8 137.4) (end 189.6 139.2) (width 0.25) (layer "B.Cu") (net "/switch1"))
 (segment (start 169.6 107.2) (end 128 107.2) (width 0.25) (layer "F.Cu") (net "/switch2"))
 (segment (start 194.6 139.4) (end 181.6 126.4) (width 0.25) (layer "F.Cu") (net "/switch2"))
 (segment (start 181.6 126.4) (end 176.4 126.4) (width 0.25) (layer "F.Cu") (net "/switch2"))
 (segment (start 174 124) (end 174 111.6) (width 0.25) (layer "F.Cu") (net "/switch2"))
 (segment (start 174 111.6) (end 169.6 107.2) (width 0.25) (layer "F.Cu") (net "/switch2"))
 (segment (start 128 107.2) (end 127.2 106.4) (width 0.25) (layer "F.Cu") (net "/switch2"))
 (segment (start 195.27 139.62) (end 194.6 139.4) (width 0.25) (layer "F.Cu") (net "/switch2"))
 (segment (start 176.4 126.4) (end 174 124) (width 0.25) (layer "F.Cu") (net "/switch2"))
 (via (at 127.2 106.4) (size 0.6) (drill 0.3) (layers "F.Cu" "B.Cu") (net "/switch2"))
 (segment (start 124.6 103.8) (end 124 103.3) (width 0.25) (layer "B.Cu") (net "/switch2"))
 (segment (start 127.2 106.4) (end 124.6 103.8) (width 0.25) (layer "B.Cu") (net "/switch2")))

